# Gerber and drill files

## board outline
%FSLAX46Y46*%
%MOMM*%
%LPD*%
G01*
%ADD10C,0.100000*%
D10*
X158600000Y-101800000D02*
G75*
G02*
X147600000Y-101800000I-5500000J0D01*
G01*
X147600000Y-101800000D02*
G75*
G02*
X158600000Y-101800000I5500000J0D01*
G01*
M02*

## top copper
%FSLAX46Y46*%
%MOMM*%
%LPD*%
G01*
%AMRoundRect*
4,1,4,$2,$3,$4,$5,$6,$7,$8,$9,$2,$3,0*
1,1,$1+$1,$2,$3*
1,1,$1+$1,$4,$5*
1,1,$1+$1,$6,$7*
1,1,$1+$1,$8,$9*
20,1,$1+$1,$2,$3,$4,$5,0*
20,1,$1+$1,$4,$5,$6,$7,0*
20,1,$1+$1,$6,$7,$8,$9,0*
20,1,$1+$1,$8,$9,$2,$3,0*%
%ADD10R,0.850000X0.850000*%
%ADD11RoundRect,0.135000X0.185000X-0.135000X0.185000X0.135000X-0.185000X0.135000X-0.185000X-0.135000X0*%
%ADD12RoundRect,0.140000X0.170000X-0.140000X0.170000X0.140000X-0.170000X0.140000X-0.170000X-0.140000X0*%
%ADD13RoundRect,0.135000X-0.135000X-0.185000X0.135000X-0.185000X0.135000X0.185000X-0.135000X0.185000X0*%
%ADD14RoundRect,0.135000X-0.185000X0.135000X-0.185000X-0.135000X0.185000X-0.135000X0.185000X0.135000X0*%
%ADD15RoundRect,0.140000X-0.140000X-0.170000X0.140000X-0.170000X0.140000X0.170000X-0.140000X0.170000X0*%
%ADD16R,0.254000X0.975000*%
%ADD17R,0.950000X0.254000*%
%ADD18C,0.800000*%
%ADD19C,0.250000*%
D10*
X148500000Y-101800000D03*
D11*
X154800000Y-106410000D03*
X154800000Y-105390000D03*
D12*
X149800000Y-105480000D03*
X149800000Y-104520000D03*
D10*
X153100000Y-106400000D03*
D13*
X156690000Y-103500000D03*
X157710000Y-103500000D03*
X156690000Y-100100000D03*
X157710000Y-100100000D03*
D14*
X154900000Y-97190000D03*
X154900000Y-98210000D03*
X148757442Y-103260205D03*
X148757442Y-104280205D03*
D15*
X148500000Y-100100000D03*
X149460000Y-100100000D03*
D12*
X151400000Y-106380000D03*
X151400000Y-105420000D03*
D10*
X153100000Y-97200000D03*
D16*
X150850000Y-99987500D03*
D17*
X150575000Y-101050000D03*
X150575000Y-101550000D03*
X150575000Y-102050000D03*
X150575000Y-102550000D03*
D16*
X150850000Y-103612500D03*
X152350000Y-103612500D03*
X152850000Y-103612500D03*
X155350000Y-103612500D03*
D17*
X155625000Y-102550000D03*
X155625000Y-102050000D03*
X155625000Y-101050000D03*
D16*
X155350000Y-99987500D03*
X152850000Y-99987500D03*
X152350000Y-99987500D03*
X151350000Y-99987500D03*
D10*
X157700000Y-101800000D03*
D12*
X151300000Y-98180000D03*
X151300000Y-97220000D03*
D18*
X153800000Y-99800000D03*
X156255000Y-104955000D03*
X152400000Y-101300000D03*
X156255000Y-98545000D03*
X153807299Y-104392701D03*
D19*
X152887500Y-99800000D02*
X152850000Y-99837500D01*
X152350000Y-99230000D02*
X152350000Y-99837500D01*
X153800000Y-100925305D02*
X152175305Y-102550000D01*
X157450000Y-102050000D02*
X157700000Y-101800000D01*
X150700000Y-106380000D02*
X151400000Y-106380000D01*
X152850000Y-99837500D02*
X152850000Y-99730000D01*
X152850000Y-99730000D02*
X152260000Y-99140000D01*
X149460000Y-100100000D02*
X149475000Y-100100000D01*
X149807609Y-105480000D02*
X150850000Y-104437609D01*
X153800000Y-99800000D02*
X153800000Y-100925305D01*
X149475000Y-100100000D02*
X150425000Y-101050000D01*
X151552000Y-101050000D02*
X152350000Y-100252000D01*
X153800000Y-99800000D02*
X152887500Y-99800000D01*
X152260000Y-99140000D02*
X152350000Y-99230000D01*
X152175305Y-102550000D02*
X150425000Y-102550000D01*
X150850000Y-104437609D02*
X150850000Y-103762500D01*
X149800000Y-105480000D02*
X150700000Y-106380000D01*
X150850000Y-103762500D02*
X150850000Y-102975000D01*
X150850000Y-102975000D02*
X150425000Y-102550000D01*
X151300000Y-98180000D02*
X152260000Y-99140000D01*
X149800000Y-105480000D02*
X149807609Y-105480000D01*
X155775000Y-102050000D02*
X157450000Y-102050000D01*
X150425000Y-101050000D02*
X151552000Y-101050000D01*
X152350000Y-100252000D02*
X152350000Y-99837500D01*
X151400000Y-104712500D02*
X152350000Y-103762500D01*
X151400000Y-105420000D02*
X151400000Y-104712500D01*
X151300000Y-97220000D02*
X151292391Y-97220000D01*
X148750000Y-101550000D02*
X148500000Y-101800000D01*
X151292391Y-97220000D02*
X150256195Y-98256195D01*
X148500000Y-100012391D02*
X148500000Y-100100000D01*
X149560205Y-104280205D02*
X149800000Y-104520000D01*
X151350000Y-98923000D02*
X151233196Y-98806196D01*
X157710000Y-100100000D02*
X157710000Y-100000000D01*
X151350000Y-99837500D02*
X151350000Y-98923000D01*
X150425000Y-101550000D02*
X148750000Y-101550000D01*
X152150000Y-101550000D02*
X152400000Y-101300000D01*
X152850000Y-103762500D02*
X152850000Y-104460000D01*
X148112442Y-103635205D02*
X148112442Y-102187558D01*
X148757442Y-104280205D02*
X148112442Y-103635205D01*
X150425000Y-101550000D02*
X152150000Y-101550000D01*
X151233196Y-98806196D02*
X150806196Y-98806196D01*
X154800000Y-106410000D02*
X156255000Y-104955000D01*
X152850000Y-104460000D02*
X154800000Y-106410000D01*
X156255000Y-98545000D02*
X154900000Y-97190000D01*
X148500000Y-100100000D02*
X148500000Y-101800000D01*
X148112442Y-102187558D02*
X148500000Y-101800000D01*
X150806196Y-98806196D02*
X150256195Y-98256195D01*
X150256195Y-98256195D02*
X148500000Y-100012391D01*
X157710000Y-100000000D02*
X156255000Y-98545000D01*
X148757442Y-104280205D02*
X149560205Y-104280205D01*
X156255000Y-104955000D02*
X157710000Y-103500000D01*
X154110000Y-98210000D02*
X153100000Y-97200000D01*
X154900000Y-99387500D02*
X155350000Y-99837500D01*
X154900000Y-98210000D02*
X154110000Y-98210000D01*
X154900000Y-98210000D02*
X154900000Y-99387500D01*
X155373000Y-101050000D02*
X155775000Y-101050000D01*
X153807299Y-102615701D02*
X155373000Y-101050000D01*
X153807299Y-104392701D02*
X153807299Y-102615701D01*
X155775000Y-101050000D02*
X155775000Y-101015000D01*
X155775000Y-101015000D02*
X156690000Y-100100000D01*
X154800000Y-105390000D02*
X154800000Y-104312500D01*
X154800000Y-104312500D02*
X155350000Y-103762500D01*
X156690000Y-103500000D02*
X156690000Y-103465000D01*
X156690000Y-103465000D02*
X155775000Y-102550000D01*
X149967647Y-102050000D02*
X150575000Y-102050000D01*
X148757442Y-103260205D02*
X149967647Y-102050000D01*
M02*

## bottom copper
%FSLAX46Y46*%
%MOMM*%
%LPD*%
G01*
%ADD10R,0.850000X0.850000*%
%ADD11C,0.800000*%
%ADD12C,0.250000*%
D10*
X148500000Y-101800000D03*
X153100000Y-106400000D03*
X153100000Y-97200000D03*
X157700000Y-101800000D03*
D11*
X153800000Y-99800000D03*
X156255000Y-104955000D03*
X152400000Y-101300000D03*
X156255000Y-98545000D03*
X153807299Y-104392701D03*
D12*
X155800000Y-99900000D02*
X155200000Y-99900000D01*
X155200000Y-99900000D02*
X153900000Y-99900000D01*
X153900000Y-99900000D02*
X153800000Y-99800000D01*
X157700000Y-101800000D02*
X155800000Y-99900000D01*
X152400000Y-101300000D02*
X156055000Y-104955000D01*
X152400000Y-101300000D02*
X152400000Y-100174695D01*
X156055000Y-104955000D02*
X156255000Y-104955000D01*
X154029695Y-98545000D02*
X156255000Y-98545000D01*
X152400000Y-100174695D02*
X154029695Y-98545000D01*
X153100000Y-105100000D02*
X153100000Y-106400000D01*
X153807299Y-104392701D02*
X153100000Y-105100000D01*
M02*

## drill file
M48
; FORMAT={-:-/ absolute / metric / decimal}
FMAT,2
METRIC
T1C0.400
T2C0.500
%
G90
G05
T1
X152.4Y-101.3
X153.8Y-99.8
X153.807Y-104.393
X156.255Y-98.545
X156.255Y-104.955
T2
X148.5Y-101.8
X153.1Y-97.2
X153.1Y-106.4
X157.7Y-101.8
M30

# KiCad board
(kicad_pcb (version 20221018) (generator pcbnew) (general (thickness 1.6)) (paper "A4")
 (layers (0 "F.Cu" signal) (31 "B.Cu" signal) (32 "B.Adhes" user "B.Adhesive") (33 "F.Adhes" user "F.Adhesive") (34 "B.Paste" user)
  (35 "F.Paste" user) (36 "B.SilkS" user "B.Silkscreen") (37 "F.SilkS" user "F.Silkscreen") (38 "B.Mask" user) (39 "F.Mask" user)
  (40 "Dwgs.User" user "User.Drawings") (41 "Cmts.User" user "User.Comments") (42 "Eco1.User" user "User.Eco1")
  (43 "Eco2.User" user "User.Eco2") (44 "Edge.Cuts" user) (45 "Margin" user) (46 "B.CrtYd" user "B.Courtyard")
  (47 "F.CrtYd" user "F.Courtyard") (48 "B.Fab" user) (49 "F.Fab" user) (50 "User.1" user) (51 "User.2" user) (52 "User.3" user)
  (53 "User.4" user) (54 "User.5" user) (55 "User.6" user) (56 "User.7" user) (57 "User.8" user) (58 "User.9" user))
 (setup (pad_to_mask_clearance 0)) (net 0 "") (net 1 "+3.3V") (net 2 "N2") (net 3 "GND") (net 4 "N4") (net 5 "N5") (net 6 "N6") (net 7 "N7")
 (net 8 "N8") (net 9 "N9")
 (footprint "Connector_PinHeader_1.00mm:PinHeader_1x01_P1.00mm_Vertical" (layer "F.Cu") (at 148.5 101.8)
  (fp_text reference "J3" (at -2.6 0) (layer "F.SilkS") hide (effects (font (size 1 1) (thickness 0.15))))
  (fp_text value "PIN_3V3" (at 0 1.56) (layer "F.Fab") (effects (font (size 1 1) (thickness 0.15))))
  (pad "1" thru_hole rect (at 0 0) (size 0.85 0.85) (drill 0.5) (layers "*.Cu" "*.Mask") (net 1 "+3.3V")))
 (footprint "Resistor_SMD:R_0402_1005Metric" (layer "F.Cu") (at 154.8 105.9 90)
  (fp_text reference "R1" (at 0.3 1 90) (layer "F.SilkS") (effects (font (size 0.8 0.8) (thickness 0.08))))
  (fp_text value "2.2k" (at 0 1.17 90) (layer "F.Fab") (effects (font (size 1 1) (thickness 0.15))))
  (pad "1" smd roundrect (at -0.51 0 90) (size 0.54 0.64) (layers "F.Cu" "F.Paste" "F.Mask") (roundrect_rratio 0.25) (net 1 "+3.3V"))
  (pad "2" smd roundrect (at 0.51 0 90) (size 0.54 0.64) (layers "F.Cu" "F.Paste" "F.Mask") (roundrect_rratio 0.25) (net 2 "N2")))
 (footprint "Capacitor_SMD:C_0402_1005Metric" (layer "F.Cu") (at 149.8 105 90)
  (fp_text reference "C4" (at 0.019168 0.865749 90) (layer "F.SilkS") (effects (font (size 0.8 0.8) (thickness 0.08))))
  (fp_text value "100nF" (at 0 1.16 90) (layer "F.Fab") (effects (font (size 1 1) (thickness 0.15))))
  (pad "1" smd roundrect (at -0.48 0 90) (size 0.56 0.62) (layers "F.Cu" "F.Paste" "F.Mask") (roundrect_rratio 0.25) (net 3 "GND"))
  (pad "2" smd roundrect (at 0.48 0 90) (size 0.56 0.62) (layers "F.Cu" "F.Paste" "F.Mask") (roundrect_rratio 0.25) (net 1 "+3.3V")))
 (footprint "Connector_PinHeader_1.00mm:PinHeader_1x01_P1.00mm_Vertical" (layer "F.Cu") (at 153.1 106.4)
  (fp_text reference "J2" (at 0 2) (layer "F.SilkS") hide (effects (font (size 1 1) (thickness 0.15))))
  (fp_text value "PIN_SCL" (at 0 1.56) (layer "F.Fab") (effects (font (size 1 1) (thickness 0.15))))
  (pad "1" thru_hole rect (at 0 0) (size 0.85 0.85) (drill 0.5) (layers "*.Cu" "*.Mask") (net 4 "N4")))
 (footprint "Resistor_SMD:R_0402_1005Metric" (layer "F.Cu") (at 157.2 103.5)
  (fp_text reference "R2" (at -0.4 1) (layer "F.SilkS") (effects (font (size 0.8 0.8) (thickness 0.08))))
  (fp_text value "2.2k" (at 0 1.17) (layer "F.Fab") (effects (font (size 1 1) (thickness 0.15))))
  (pad "1" smd roundrect (at -0.51 0) (size 0.54 0.64) (layers "F.Cu" "F.Paste" "F.Mask") (roundrect_rratio 0.25) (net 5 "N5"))
  (pad "2" smd roundrect (at 0.51 0) (size 0.54 0.64) (layers "F.Cu" "F.Paste" "F.Mask") (roundrect_rratio 0.25) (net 1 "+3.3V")))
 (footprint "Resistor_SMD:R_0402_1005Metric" (layer "F.Cu") (at 157.2 100.1)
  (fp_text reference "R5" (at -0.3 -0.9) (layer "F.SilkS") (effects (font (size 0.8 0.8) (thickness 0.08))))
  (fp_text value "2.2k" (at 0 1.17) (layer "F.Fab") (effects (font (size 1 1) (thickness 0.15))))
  (pad "1" smd roundrect (at -0.51 0) (size 0.54 0.64) (layers "F.Cu" "F.Paste" "F.Mask") (roundrect_rratio 0.25) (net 4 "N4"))
  (pad "2" smd roundrect (at 0.51 0) (size 0.54 0.64) (layers "F.Cu" "F.Paste" "F.Mask") (roundrect_rratio 0.25) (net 1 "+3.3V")))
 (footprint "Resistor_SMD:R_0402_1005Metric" (layer "F.Cu") (at 154.9 97.7 -90)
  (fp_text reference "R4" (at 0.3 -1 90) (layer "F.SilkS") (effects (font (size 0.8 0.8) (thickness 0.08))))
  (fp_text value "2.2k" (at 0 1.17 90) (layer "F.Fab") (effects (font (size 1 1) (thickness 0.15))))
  (pad "1" smd roundrect (at -0.51 0 270) (size 0.54 0.64) (layers "F.Cu" "F.Paste" "F.Mask") (roundrect_rratio 0.25) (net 1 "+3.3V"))
  (pad "2" smd roundrect (at 0.51 0 270) (size 0.54 0.64) (layers "F.Cu" "F.Paste" "F.Mask") (roundrect_rratio 0.25) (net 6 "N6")))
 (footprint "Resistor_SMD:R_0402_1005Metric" (layer "F.Cu") (at 148.757442 103.770205 -90)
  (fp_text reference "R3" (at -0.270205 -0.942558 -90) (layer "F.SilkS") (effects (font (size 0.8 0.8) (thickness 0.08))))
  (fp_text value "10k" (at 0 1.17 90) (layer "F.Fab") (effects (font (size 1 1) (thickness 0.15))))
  (pad "1" smd roundrect (at -0.51 0 270) (size 0.54 0.64) (layers "F.Cu" "F.Paste" "F.Mask") (roundrect_rratio 0.25) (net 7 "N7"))
  (pad "2" smd roundrect (at 0.51 0 270) (size 0.54 0.64) (layers "F.Cu" "F.Paste" "F.Mask") (roundrect_rratio 0.25) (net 1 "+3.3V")))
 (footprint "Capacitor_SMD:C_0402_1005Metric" (layer "F.Cu") (at 148.98 100.1)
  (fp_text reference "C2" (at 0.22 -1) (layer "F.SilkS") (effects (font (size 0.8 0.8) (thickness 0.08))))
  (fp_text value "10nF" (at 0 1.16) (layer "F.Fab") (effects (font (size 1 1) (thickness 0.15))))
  (pad "1" smd roundrect (at -0.48 0) (size 0.56 0.62) (layers "F.Cu" "F.Paste" "F.Mask") (roundrect_rratio 0.25) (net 1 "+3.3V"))
  (pad "2" smd roundrect (at 0.48 0) (size 0.56 0.62) (layers "F.Cu" "F.Paste" "F.Mask") (roundrect_rratio 0.25) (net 3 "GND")))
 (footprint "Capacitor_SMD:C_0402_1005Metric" (layer "F.Cu") (at 151.4 105.9 90)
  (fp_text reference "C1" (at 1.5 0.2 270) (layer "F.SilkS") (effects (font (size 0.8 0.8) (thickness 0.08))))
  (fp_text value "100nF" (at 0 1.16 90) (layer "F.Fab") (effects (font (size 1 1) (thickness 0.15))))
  (pad "1" smd roundrect (at -0.48 0 90) (size 0.56 0.62) (layers "F.Cu" "F.Paste" "F.Mask") (roundrect_rratio 0.25) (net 3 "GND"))
  (pad "2" smd roundrect (at 0.48 0 90) (size 0.56 0.62) (layers "F.Cu" "F.Paste" "F.Mask") (roundrect_rratio 0.25) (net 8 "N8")))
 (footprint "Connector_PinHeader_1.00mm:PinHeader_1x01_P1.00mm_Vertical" (layer "F.Cu") (at 153.1 97.2)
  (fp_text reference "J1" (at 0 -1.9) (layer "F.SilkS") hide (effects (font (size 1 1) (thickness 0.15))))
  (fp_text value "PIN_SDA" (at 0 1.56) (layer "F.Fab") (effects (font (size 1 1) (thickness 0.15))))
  (pad "1" thru_hole rect (at 0 0) (size 0.85 0.85) (drill 0.5) (layers "*.Cu" "*.Mask") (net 6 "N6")))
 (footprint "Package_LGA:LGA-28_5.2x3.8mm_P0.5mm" (layer "F.Cu") (at 153.1 101.8)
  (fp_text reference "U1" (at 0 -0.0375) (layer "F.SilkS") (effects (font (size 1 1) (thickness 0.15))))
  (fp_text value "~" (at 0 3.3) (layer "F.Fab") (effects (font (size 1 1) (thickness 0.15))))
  (pad "1" smd rect (at -2.25 -1.8125) (size 0.254 0.975) (layers "F.Cu" "F.Paste" "F.Mask") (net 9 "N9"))
  (pad "2" smd rect (at -2.525 -0.75 90) (size 0.254 0.95) (layers "F.Cu" "F.Paste" "F.Mask") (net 3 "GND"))
  (pad "3" smd rect (at -2.525 -0.25 90) (size 0.254 0.95) (layers "F.Cu" "F.Paste" "F.Mask") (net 1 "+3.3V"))
  (pad "4" smd rect (at -2.525 0.25 90) (size 0.254 0.95) (layers "F.Cu" "F.Paste" "F.Mask") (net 7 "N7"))
  (pad "5" smd rect (at -2.525 0.75 90) (size 0.254 0.95) (layers "F.Cu" "F.Paste" "F.Mask") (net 3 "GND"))
  (pad "6" smd rect (at -2.25 1.8125) (size 0.254 0.975) (layers "F.Cu" "F.Paste" "F.Mask") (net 3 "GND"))
  (pad "9" smd rect (at -0.75 1.8125) (size 0.254 0.975) (layers "F.Cu" "F.Paste" "F.Mask") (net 8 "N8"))
  (pad "10" smd rect (at -0.25 1.8125) (size 0.254 0.975) (layers "F.Cu" "F.Paste" "F.Mask") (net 1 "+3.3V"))
  (pad "15" smd rect (at 2.25 1.8125) (size 0.254 0.975) (layers "F.Cu" "F.Paste" "F.Mask") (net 2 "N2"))
  (pad "16" smd rect (at 2.525 0.75 90) (size 0.254 0.95) (layers "F.Cu" "F.Paste" "F.Mask") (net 5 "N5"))
  (pad "17" smd rect (at 2.525 0.25 90) (size 0.254 0.95) (layers "F.Cu" "F.Paste" "F.Mask") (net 3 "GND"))
  (pad "19" smd rect (at 2.525 -0.75 90) (size 0.254 0.95) (layers "F.Cu" "F.Paste" "F.Mask") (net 4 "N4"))
  (pad "20" smd rect (at 2.25 -1.8125) (size 0.254 0.975) (layers "F.Cu" "F.Paste" "F.Mask") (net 6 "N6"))
  (pad "25" smd rect (at -0.25 -1.8125) (size 0.254 0.975) (layers "F.Cu" "F.Paste" "F.Mask") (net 3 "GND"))
  (pad "26" smd rect (at -0.75 -1.8125) (size 0.254 0.975) (layers "F.Cu" "F.Paste" "F.Mask") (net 3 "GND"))
  (pad "28" smd rect (at -1.75 -1.8125) (size 0.254 0.975) (layers "F.Cu" "F.Paste" "F.Mask") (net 1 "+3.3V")))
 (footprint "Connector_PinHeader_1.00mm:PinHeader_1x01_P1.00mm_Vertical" (layer "F.Cu") (at 157.7 101.8)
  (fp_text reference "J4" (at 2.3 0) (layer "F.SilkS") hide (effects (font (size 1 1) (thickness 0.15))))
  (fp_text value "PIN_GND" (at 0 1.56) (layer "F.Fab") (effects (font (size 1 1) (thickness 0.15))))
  (pad "1" thru_hole rect (at 0 0) (size 0.85 0.85) (drill 0.5) (layers "*.Cu" "*.Mask") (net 3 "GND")))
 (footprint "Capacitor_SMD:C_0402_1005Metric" (layer "F.Cu") (at 151.3 97.7 90)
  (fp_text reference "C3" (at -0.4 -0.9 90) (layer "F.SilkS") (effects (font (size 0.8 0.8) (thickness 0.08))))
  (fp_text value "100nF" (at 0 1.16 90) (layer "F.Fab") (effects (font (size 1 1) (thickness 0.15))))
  (pad "1" smd roundrect (at -0.48 0 90) (size 0.56 0.62) (layers "F.Cu" "F.Paste" "F.Mask") (roundrect_rratio 0.25) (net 3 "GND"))
  (pad "2" smd roundrect (at 0.48 0 90) (size 0.56 0.62) (layers "F.Cu" "F.Paste" "F.Mask") (roundrect_rratio 0.25) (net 1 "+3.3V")))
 (gr_circle (center 153.1 101.8) (end 158.6 101.8) (stroke (width 0.1) (type default)) (fill none) (layer "Edge.Cuts"))
 (segment (start 152.8875 99.8) (end 152.85 99.8375) (width 0.25) (layer "F.Cu") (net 3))
 (segment (start 152.35 99.23) (end 152.35 99.8375) (width 0.25) (layer "F.Cu") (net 3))
 (segment (start 153.8 100.925305) (end 152.175305 102.55) (width 0.25) (layer "F.Cu") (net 3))
 (segment (start 157.45 102.05) (end 157.7 101.8) (width 0.25) (layer "F.Cu") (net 3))
 (segment (start 150.7 106.38) (end 151.4 106.38) (width 0.25) (layer "F.Cu") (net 3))
 (segment (start 152.85 99.8375) (end 152.85 99.73) (width 0.25) (layer "F.Cu") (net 3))
 (segment (start 152.85 99.73) (end 152.26 99.14) (width 0.25) (layer "F.Cu") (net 3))
 (segment (start 149.46 100.1) (end 149.475 100.1) (width 0.25) (layer "F.Cu") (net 3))
 (segment (start 149.807609 105.48) (end 150.85 104.437609) (width 0.25) (layer "F.Cu") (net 3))
 (segment (start 153.8 99.8) (end 153.8 100.925305) (width 0.25) (layer "F.Cu") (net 3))
 (segment (start 149.475 100.1) (end 150.425 101.05) (width 0.25) (layer "F.Cu") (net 3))
 (segment (start 151.552 101.05) (end 152.35 100.252) (width 0.25) (layer "F.Cu") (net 3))
 (segment (start 153.8 99.8) (end 152.8875 99.8) (width 0.25) (layer "F.Cu") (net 3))
 (segment (start 152.26 99.14) (end 152.35 99.23) (width 0.25) (layer "F.Cu") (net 3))
 (segment (start 152.175305 102.55) (end 150.425 102.55) (width 0.25) (layer "F.Cu") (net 3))
 (segment (start 150.85 104.437609) (end 150.85 103.7625) (width 0.25) (layer "F.Cu") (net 3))
 (segment (start 149.8 105.48) (end 150.7 106.38) (width 0.25) (layer "F.Cu") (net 3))
 (segment (start 150.85 103.7625) (end 150.85 102.975) (width 0.25) (layer "F.Cu") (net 3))
 (segment (start 150.85 102.975) (end 150.425 102.55) (width 0.25) (layer "F.Cu") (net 3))
 (segment (start 151.3 98.18) (end 152.26 99.14) (width 0.25) (layer "F.Cu") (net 3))
 (segment (start 149.8 105.48) (end 149.807609 105.48) (width 0.25) (layer "F.Cu") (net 3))
 (segment (start 155.775 102.05) (end 157.45 102.05) (width 0.25) (layer "F.Cu") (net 3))
 (segment (start 150.425 101.05) (end 151.552 101.05) (width 0.25) (layer "F.Cu") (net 3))
 (segment (start 152.35 100.252) (end 152.35 99.8375) (width 0.25) (layer "F.Cu") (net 3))
 (via (at 153.8 99.8) (size 0.8) (drill 0.4) (layers "F.Cu" "B.Cu") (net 3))
 (segment (start 155.8 99.9) (end 155.2 99.9) (width 0.25) (layer "B.Cu") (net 3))
 (segment (start 155.2 99.9) (end 153.9 99.9) (width 0.25) (layer "B.Cu") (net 3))
 (segment (start 153.9 99.9) (end 153.8 99.8) (width 0.25) (layer "B.Cu") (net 3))
 (segment (start 157.7 101.8) (end 155.8 99.9) (width 0.25) (layer "B.Cu") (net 3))
 (segment (start 151.4 104.7125) (end 152.35 103.7625) (width 0.25) (layer "F.Cu") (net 8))
 (segment (start 151.4 105.42) (end 151.4 104.7125) (width 0.25) (layer "F.Cu") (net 8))
 (segment (start 151.3 97.22) (end 151.292391 97.22) (width 0.25) (layer "F.Cu") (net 1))
 (segment (start 148.75 101.55) (end 148.5 101.8) (width 0.25) (layer "F.Cu") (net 1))
 (segment (start 151.292391 97.22) (end 150.256195 98.256195) (width 0.25) (layer "F.Cu") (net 1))
 (segment (start 148.5 100.012391) (end 148.5 100.1) (width 0.25) (layer "F.Cu") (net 1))
 (segment (start 149.560205 104.280205) (end 149.8 104.52) (width 0.25) (layer "F.Cu") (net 1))
 (segment (start 151.35 98.923) (end 151.233196 98.806196) (width 0.25) (layer "F.Cu") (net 1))
 (segment (start 157.71 100.1) (end 157.71 100) (width 0.25) (layer "F.Cu") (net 1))
 (segment (start 151.35 99.8375) (end 151.35 98.923) (width 0.25) (layer "F.Cu") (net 1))
 (segment (start 150.425 101.55) (end 148.75 101.55) (width 0.25) (layer "F.Cu") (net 1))
 (segment (start 152.15 101.55) (end 152.4 101.3) (width 0.25) (layer "F.Cu") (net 1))
 (segment (start 152.85 103.7625) (end 152.85 104.46) (width 0.25) (layer "F.Cu") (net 1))
 (segment (start 148.112442 103.635205) (end 148.112442 102.187558) (width 0.25) (layer "F.Cu") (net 1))
 (segment (start 148.757442 104.280205) (end 148.112442 103.635205) (width 0.25) (layer "F.Cu") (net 1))
 (segment (start 150.425 101.55) (end 152.15 101.55) (width 0.25) (layer "F.Cu") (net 1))
 (segment (start 151.233196 98.806196) (end 150.806196 98.806196) (width 0.25) (layer "F.Cu") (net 1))
 (segment (start 154.8 106.41) (end 156.255 104.955) (width 0.25) (layer "F.Cu") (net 1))
 (segment (start 152.85 104.46) (end 154.8 106.41) (width 0.25) (layer "F.Cu") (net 1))
 (segment (start 156.255 98.545) (end 154.9 97.19) (width 0.25) (layer "F.Cu") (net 1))
 (segment (start 148.5 100.1) (end 148.5 101.8) (width 0.25) (layer "F.Cu") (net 1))
 (segment (start 148.112442 102.187558) (end 148.5 101.8) (width 0.25) (layer "F.Cu") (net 1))
 (segment (start 150.806196 98.806196) (end 150.256195 98.256195) (width 0.25) (layer "F.Cu") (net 1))
 (segment (start 150.256195 98.256195) (end 148.5 100.012391) (width 0.25) (layer "F.Cu") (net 1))
 (segment (start 157.71 100) (end 156.255 98.545) (width 0.25) (layer "F.Cu") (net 1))
 (segment (start 148.757442 104.280205) (end 149.560205 104.280205) (width 0.25) (layer "F.Cu") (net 1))
 (segment (start 156.255 104.955) (end 157.71 103.5) (width 0.25) (layer "F.Cu") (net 1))
 (via (at 156.255 104.955) (size 0.8) (drill 0.4) (layers "F.Cu" "B.Cu") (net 1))
 (via (at 152.4 101.3) (size 0.8) (drill 0.4) (layers "F.Cu" "B.Cu") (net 1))
 (via (at 156.255 98.545) (size 0.8) (drill 0.4) (layers "F.Cu" "B.Cu") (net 1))
 (segment (start 152.4 101.3) (end 156.055 104.955) (width 0.25) (layer "B.Cu") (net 1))
 (segment (start 152.4 101.3) (end 152.4 100.174695) (width 0.25) (layer "B.Cu") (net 1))
 (segment (start 156.055 104.955) (end 156.255 104.955) (width 0.25) (layer "B.Cu") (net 1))
 (segment (start 154.029695 98.545) (end 156.255 98.545) (width 0.25) (layer "B.Cu") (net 1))
 (segment (start 152.4 100.174695) (end 154.029695 98.545) (width 0.25) (layer "B.Cu") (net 1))
 (segment (start 154.11 98.21) (end 153.1 97.2) (width 0.25) (layer "F.Cu") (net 6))
 (segment (start 154.9 99.3875) (end 155.35 99.8375) (width 0.25) (layer "F.Cu") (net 6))
 (segment (start 154.9 98.21) (end 154.11 98.21) (width 0.25) (layer "F.Cu") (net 6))
 (segment (start 154.9 98.21) (end 154.9 99.3875) (width 0.25) (layer "F.Cu") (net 6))
 (segment (start 155.373 101.05) (end 155.775 101.05) (width 0.25) (layer "F.Cu") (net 4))
 (segment (start 153.807299 102.615701) (end 155.373 101.05) (width 0.25) (layer "F.Cu") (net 4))
 (segment (start 153.807299 104.392701) (end 153.807299 102.615701) (width 0.25) (layer "F.Cu") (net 4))
 (segment (start 155.775 101.05) (end 155.775 101.015) (width 0.25) (layer "F.Cu") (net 4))
 (segment (start 155.775 101.015) (end 156.69 100.1) (width 0.25) (layer "F.Cu") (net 4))
 (via (at 153.807299 104.392701) (size 0.8) (drill 0.4) (layers "F.Cu" "B.Cu") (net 4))
 (segment (start 153.1 105.1) (end 153.1 106.4) (width 0.25) (layer "B.Cu") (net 4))
 (segment (start 153.807299 104.392701) (end 153.1 105.1) (width 0.25) (layer "B.Cu") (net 4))
 (segment (start 154.8 105.39) (end 154.8 104.3125) (width 0.25) (layer "F.Cu") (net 2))
 (segment (start 154.8 104.3125) (end 155.35 103.7625) (width 0.25) (layer "F.Cu") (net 2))
 (segment (start 156.69 103.5) (end 156.69 103.465) (width 0.25) (layer "F.Cu") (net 5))
 (segment (start 156.69 103.465) (end 155.775 102.55) (width 0.25) (layer "F.Cu") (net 5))
 (segment (start 149.967647 102.05) (end 150.575 102.05) (width 0.25) (layer "F.Cu") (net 7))
 (segment (start 148.757442 103.260205) (end 149.967647 102.05) (width 0.25) (layer "F.Cu") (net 7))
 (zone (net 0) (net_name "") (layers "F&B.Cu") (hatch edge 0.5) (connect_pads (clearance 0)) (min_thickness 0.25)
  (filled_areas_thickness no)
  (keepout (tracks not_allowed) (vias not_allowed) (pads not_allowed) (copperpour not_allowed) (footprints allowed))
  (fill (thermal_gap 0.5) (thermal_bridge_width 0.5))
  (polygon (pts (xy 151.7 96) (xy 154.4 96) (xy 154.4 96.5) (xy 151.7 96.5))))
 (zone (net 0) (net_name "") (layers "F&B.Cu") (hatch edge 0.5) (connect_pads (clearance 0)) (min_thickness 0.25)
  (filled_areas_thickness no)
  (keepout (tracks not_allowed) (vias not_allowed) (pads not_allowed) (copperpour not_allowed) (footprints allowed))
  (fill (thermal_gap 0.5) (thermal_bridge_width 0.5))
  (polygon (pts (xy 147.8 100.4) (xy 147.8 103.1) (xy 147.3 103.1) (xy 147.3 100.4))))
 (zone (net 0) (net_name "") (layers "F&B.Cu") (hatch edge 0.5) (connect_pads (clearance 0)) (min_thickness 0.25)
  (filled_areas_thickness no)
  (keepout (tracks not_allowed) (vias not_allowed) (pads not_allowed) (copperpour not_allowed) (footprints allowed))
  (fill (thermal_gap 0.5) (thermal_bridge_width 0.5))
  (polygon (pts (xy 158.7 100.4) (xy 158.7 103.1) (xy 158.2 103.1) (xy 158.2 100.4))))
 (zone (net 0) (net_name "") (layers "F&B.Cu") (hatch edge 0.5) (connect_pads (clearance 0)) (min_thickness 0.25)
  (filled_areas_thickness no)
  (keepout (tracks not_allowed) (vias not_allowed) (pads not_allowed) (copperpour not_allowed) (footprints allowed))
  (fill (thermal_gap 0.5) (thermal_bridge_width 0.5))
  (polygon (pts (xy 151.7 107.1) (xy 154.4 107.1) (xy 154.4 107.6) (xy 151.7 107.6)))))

